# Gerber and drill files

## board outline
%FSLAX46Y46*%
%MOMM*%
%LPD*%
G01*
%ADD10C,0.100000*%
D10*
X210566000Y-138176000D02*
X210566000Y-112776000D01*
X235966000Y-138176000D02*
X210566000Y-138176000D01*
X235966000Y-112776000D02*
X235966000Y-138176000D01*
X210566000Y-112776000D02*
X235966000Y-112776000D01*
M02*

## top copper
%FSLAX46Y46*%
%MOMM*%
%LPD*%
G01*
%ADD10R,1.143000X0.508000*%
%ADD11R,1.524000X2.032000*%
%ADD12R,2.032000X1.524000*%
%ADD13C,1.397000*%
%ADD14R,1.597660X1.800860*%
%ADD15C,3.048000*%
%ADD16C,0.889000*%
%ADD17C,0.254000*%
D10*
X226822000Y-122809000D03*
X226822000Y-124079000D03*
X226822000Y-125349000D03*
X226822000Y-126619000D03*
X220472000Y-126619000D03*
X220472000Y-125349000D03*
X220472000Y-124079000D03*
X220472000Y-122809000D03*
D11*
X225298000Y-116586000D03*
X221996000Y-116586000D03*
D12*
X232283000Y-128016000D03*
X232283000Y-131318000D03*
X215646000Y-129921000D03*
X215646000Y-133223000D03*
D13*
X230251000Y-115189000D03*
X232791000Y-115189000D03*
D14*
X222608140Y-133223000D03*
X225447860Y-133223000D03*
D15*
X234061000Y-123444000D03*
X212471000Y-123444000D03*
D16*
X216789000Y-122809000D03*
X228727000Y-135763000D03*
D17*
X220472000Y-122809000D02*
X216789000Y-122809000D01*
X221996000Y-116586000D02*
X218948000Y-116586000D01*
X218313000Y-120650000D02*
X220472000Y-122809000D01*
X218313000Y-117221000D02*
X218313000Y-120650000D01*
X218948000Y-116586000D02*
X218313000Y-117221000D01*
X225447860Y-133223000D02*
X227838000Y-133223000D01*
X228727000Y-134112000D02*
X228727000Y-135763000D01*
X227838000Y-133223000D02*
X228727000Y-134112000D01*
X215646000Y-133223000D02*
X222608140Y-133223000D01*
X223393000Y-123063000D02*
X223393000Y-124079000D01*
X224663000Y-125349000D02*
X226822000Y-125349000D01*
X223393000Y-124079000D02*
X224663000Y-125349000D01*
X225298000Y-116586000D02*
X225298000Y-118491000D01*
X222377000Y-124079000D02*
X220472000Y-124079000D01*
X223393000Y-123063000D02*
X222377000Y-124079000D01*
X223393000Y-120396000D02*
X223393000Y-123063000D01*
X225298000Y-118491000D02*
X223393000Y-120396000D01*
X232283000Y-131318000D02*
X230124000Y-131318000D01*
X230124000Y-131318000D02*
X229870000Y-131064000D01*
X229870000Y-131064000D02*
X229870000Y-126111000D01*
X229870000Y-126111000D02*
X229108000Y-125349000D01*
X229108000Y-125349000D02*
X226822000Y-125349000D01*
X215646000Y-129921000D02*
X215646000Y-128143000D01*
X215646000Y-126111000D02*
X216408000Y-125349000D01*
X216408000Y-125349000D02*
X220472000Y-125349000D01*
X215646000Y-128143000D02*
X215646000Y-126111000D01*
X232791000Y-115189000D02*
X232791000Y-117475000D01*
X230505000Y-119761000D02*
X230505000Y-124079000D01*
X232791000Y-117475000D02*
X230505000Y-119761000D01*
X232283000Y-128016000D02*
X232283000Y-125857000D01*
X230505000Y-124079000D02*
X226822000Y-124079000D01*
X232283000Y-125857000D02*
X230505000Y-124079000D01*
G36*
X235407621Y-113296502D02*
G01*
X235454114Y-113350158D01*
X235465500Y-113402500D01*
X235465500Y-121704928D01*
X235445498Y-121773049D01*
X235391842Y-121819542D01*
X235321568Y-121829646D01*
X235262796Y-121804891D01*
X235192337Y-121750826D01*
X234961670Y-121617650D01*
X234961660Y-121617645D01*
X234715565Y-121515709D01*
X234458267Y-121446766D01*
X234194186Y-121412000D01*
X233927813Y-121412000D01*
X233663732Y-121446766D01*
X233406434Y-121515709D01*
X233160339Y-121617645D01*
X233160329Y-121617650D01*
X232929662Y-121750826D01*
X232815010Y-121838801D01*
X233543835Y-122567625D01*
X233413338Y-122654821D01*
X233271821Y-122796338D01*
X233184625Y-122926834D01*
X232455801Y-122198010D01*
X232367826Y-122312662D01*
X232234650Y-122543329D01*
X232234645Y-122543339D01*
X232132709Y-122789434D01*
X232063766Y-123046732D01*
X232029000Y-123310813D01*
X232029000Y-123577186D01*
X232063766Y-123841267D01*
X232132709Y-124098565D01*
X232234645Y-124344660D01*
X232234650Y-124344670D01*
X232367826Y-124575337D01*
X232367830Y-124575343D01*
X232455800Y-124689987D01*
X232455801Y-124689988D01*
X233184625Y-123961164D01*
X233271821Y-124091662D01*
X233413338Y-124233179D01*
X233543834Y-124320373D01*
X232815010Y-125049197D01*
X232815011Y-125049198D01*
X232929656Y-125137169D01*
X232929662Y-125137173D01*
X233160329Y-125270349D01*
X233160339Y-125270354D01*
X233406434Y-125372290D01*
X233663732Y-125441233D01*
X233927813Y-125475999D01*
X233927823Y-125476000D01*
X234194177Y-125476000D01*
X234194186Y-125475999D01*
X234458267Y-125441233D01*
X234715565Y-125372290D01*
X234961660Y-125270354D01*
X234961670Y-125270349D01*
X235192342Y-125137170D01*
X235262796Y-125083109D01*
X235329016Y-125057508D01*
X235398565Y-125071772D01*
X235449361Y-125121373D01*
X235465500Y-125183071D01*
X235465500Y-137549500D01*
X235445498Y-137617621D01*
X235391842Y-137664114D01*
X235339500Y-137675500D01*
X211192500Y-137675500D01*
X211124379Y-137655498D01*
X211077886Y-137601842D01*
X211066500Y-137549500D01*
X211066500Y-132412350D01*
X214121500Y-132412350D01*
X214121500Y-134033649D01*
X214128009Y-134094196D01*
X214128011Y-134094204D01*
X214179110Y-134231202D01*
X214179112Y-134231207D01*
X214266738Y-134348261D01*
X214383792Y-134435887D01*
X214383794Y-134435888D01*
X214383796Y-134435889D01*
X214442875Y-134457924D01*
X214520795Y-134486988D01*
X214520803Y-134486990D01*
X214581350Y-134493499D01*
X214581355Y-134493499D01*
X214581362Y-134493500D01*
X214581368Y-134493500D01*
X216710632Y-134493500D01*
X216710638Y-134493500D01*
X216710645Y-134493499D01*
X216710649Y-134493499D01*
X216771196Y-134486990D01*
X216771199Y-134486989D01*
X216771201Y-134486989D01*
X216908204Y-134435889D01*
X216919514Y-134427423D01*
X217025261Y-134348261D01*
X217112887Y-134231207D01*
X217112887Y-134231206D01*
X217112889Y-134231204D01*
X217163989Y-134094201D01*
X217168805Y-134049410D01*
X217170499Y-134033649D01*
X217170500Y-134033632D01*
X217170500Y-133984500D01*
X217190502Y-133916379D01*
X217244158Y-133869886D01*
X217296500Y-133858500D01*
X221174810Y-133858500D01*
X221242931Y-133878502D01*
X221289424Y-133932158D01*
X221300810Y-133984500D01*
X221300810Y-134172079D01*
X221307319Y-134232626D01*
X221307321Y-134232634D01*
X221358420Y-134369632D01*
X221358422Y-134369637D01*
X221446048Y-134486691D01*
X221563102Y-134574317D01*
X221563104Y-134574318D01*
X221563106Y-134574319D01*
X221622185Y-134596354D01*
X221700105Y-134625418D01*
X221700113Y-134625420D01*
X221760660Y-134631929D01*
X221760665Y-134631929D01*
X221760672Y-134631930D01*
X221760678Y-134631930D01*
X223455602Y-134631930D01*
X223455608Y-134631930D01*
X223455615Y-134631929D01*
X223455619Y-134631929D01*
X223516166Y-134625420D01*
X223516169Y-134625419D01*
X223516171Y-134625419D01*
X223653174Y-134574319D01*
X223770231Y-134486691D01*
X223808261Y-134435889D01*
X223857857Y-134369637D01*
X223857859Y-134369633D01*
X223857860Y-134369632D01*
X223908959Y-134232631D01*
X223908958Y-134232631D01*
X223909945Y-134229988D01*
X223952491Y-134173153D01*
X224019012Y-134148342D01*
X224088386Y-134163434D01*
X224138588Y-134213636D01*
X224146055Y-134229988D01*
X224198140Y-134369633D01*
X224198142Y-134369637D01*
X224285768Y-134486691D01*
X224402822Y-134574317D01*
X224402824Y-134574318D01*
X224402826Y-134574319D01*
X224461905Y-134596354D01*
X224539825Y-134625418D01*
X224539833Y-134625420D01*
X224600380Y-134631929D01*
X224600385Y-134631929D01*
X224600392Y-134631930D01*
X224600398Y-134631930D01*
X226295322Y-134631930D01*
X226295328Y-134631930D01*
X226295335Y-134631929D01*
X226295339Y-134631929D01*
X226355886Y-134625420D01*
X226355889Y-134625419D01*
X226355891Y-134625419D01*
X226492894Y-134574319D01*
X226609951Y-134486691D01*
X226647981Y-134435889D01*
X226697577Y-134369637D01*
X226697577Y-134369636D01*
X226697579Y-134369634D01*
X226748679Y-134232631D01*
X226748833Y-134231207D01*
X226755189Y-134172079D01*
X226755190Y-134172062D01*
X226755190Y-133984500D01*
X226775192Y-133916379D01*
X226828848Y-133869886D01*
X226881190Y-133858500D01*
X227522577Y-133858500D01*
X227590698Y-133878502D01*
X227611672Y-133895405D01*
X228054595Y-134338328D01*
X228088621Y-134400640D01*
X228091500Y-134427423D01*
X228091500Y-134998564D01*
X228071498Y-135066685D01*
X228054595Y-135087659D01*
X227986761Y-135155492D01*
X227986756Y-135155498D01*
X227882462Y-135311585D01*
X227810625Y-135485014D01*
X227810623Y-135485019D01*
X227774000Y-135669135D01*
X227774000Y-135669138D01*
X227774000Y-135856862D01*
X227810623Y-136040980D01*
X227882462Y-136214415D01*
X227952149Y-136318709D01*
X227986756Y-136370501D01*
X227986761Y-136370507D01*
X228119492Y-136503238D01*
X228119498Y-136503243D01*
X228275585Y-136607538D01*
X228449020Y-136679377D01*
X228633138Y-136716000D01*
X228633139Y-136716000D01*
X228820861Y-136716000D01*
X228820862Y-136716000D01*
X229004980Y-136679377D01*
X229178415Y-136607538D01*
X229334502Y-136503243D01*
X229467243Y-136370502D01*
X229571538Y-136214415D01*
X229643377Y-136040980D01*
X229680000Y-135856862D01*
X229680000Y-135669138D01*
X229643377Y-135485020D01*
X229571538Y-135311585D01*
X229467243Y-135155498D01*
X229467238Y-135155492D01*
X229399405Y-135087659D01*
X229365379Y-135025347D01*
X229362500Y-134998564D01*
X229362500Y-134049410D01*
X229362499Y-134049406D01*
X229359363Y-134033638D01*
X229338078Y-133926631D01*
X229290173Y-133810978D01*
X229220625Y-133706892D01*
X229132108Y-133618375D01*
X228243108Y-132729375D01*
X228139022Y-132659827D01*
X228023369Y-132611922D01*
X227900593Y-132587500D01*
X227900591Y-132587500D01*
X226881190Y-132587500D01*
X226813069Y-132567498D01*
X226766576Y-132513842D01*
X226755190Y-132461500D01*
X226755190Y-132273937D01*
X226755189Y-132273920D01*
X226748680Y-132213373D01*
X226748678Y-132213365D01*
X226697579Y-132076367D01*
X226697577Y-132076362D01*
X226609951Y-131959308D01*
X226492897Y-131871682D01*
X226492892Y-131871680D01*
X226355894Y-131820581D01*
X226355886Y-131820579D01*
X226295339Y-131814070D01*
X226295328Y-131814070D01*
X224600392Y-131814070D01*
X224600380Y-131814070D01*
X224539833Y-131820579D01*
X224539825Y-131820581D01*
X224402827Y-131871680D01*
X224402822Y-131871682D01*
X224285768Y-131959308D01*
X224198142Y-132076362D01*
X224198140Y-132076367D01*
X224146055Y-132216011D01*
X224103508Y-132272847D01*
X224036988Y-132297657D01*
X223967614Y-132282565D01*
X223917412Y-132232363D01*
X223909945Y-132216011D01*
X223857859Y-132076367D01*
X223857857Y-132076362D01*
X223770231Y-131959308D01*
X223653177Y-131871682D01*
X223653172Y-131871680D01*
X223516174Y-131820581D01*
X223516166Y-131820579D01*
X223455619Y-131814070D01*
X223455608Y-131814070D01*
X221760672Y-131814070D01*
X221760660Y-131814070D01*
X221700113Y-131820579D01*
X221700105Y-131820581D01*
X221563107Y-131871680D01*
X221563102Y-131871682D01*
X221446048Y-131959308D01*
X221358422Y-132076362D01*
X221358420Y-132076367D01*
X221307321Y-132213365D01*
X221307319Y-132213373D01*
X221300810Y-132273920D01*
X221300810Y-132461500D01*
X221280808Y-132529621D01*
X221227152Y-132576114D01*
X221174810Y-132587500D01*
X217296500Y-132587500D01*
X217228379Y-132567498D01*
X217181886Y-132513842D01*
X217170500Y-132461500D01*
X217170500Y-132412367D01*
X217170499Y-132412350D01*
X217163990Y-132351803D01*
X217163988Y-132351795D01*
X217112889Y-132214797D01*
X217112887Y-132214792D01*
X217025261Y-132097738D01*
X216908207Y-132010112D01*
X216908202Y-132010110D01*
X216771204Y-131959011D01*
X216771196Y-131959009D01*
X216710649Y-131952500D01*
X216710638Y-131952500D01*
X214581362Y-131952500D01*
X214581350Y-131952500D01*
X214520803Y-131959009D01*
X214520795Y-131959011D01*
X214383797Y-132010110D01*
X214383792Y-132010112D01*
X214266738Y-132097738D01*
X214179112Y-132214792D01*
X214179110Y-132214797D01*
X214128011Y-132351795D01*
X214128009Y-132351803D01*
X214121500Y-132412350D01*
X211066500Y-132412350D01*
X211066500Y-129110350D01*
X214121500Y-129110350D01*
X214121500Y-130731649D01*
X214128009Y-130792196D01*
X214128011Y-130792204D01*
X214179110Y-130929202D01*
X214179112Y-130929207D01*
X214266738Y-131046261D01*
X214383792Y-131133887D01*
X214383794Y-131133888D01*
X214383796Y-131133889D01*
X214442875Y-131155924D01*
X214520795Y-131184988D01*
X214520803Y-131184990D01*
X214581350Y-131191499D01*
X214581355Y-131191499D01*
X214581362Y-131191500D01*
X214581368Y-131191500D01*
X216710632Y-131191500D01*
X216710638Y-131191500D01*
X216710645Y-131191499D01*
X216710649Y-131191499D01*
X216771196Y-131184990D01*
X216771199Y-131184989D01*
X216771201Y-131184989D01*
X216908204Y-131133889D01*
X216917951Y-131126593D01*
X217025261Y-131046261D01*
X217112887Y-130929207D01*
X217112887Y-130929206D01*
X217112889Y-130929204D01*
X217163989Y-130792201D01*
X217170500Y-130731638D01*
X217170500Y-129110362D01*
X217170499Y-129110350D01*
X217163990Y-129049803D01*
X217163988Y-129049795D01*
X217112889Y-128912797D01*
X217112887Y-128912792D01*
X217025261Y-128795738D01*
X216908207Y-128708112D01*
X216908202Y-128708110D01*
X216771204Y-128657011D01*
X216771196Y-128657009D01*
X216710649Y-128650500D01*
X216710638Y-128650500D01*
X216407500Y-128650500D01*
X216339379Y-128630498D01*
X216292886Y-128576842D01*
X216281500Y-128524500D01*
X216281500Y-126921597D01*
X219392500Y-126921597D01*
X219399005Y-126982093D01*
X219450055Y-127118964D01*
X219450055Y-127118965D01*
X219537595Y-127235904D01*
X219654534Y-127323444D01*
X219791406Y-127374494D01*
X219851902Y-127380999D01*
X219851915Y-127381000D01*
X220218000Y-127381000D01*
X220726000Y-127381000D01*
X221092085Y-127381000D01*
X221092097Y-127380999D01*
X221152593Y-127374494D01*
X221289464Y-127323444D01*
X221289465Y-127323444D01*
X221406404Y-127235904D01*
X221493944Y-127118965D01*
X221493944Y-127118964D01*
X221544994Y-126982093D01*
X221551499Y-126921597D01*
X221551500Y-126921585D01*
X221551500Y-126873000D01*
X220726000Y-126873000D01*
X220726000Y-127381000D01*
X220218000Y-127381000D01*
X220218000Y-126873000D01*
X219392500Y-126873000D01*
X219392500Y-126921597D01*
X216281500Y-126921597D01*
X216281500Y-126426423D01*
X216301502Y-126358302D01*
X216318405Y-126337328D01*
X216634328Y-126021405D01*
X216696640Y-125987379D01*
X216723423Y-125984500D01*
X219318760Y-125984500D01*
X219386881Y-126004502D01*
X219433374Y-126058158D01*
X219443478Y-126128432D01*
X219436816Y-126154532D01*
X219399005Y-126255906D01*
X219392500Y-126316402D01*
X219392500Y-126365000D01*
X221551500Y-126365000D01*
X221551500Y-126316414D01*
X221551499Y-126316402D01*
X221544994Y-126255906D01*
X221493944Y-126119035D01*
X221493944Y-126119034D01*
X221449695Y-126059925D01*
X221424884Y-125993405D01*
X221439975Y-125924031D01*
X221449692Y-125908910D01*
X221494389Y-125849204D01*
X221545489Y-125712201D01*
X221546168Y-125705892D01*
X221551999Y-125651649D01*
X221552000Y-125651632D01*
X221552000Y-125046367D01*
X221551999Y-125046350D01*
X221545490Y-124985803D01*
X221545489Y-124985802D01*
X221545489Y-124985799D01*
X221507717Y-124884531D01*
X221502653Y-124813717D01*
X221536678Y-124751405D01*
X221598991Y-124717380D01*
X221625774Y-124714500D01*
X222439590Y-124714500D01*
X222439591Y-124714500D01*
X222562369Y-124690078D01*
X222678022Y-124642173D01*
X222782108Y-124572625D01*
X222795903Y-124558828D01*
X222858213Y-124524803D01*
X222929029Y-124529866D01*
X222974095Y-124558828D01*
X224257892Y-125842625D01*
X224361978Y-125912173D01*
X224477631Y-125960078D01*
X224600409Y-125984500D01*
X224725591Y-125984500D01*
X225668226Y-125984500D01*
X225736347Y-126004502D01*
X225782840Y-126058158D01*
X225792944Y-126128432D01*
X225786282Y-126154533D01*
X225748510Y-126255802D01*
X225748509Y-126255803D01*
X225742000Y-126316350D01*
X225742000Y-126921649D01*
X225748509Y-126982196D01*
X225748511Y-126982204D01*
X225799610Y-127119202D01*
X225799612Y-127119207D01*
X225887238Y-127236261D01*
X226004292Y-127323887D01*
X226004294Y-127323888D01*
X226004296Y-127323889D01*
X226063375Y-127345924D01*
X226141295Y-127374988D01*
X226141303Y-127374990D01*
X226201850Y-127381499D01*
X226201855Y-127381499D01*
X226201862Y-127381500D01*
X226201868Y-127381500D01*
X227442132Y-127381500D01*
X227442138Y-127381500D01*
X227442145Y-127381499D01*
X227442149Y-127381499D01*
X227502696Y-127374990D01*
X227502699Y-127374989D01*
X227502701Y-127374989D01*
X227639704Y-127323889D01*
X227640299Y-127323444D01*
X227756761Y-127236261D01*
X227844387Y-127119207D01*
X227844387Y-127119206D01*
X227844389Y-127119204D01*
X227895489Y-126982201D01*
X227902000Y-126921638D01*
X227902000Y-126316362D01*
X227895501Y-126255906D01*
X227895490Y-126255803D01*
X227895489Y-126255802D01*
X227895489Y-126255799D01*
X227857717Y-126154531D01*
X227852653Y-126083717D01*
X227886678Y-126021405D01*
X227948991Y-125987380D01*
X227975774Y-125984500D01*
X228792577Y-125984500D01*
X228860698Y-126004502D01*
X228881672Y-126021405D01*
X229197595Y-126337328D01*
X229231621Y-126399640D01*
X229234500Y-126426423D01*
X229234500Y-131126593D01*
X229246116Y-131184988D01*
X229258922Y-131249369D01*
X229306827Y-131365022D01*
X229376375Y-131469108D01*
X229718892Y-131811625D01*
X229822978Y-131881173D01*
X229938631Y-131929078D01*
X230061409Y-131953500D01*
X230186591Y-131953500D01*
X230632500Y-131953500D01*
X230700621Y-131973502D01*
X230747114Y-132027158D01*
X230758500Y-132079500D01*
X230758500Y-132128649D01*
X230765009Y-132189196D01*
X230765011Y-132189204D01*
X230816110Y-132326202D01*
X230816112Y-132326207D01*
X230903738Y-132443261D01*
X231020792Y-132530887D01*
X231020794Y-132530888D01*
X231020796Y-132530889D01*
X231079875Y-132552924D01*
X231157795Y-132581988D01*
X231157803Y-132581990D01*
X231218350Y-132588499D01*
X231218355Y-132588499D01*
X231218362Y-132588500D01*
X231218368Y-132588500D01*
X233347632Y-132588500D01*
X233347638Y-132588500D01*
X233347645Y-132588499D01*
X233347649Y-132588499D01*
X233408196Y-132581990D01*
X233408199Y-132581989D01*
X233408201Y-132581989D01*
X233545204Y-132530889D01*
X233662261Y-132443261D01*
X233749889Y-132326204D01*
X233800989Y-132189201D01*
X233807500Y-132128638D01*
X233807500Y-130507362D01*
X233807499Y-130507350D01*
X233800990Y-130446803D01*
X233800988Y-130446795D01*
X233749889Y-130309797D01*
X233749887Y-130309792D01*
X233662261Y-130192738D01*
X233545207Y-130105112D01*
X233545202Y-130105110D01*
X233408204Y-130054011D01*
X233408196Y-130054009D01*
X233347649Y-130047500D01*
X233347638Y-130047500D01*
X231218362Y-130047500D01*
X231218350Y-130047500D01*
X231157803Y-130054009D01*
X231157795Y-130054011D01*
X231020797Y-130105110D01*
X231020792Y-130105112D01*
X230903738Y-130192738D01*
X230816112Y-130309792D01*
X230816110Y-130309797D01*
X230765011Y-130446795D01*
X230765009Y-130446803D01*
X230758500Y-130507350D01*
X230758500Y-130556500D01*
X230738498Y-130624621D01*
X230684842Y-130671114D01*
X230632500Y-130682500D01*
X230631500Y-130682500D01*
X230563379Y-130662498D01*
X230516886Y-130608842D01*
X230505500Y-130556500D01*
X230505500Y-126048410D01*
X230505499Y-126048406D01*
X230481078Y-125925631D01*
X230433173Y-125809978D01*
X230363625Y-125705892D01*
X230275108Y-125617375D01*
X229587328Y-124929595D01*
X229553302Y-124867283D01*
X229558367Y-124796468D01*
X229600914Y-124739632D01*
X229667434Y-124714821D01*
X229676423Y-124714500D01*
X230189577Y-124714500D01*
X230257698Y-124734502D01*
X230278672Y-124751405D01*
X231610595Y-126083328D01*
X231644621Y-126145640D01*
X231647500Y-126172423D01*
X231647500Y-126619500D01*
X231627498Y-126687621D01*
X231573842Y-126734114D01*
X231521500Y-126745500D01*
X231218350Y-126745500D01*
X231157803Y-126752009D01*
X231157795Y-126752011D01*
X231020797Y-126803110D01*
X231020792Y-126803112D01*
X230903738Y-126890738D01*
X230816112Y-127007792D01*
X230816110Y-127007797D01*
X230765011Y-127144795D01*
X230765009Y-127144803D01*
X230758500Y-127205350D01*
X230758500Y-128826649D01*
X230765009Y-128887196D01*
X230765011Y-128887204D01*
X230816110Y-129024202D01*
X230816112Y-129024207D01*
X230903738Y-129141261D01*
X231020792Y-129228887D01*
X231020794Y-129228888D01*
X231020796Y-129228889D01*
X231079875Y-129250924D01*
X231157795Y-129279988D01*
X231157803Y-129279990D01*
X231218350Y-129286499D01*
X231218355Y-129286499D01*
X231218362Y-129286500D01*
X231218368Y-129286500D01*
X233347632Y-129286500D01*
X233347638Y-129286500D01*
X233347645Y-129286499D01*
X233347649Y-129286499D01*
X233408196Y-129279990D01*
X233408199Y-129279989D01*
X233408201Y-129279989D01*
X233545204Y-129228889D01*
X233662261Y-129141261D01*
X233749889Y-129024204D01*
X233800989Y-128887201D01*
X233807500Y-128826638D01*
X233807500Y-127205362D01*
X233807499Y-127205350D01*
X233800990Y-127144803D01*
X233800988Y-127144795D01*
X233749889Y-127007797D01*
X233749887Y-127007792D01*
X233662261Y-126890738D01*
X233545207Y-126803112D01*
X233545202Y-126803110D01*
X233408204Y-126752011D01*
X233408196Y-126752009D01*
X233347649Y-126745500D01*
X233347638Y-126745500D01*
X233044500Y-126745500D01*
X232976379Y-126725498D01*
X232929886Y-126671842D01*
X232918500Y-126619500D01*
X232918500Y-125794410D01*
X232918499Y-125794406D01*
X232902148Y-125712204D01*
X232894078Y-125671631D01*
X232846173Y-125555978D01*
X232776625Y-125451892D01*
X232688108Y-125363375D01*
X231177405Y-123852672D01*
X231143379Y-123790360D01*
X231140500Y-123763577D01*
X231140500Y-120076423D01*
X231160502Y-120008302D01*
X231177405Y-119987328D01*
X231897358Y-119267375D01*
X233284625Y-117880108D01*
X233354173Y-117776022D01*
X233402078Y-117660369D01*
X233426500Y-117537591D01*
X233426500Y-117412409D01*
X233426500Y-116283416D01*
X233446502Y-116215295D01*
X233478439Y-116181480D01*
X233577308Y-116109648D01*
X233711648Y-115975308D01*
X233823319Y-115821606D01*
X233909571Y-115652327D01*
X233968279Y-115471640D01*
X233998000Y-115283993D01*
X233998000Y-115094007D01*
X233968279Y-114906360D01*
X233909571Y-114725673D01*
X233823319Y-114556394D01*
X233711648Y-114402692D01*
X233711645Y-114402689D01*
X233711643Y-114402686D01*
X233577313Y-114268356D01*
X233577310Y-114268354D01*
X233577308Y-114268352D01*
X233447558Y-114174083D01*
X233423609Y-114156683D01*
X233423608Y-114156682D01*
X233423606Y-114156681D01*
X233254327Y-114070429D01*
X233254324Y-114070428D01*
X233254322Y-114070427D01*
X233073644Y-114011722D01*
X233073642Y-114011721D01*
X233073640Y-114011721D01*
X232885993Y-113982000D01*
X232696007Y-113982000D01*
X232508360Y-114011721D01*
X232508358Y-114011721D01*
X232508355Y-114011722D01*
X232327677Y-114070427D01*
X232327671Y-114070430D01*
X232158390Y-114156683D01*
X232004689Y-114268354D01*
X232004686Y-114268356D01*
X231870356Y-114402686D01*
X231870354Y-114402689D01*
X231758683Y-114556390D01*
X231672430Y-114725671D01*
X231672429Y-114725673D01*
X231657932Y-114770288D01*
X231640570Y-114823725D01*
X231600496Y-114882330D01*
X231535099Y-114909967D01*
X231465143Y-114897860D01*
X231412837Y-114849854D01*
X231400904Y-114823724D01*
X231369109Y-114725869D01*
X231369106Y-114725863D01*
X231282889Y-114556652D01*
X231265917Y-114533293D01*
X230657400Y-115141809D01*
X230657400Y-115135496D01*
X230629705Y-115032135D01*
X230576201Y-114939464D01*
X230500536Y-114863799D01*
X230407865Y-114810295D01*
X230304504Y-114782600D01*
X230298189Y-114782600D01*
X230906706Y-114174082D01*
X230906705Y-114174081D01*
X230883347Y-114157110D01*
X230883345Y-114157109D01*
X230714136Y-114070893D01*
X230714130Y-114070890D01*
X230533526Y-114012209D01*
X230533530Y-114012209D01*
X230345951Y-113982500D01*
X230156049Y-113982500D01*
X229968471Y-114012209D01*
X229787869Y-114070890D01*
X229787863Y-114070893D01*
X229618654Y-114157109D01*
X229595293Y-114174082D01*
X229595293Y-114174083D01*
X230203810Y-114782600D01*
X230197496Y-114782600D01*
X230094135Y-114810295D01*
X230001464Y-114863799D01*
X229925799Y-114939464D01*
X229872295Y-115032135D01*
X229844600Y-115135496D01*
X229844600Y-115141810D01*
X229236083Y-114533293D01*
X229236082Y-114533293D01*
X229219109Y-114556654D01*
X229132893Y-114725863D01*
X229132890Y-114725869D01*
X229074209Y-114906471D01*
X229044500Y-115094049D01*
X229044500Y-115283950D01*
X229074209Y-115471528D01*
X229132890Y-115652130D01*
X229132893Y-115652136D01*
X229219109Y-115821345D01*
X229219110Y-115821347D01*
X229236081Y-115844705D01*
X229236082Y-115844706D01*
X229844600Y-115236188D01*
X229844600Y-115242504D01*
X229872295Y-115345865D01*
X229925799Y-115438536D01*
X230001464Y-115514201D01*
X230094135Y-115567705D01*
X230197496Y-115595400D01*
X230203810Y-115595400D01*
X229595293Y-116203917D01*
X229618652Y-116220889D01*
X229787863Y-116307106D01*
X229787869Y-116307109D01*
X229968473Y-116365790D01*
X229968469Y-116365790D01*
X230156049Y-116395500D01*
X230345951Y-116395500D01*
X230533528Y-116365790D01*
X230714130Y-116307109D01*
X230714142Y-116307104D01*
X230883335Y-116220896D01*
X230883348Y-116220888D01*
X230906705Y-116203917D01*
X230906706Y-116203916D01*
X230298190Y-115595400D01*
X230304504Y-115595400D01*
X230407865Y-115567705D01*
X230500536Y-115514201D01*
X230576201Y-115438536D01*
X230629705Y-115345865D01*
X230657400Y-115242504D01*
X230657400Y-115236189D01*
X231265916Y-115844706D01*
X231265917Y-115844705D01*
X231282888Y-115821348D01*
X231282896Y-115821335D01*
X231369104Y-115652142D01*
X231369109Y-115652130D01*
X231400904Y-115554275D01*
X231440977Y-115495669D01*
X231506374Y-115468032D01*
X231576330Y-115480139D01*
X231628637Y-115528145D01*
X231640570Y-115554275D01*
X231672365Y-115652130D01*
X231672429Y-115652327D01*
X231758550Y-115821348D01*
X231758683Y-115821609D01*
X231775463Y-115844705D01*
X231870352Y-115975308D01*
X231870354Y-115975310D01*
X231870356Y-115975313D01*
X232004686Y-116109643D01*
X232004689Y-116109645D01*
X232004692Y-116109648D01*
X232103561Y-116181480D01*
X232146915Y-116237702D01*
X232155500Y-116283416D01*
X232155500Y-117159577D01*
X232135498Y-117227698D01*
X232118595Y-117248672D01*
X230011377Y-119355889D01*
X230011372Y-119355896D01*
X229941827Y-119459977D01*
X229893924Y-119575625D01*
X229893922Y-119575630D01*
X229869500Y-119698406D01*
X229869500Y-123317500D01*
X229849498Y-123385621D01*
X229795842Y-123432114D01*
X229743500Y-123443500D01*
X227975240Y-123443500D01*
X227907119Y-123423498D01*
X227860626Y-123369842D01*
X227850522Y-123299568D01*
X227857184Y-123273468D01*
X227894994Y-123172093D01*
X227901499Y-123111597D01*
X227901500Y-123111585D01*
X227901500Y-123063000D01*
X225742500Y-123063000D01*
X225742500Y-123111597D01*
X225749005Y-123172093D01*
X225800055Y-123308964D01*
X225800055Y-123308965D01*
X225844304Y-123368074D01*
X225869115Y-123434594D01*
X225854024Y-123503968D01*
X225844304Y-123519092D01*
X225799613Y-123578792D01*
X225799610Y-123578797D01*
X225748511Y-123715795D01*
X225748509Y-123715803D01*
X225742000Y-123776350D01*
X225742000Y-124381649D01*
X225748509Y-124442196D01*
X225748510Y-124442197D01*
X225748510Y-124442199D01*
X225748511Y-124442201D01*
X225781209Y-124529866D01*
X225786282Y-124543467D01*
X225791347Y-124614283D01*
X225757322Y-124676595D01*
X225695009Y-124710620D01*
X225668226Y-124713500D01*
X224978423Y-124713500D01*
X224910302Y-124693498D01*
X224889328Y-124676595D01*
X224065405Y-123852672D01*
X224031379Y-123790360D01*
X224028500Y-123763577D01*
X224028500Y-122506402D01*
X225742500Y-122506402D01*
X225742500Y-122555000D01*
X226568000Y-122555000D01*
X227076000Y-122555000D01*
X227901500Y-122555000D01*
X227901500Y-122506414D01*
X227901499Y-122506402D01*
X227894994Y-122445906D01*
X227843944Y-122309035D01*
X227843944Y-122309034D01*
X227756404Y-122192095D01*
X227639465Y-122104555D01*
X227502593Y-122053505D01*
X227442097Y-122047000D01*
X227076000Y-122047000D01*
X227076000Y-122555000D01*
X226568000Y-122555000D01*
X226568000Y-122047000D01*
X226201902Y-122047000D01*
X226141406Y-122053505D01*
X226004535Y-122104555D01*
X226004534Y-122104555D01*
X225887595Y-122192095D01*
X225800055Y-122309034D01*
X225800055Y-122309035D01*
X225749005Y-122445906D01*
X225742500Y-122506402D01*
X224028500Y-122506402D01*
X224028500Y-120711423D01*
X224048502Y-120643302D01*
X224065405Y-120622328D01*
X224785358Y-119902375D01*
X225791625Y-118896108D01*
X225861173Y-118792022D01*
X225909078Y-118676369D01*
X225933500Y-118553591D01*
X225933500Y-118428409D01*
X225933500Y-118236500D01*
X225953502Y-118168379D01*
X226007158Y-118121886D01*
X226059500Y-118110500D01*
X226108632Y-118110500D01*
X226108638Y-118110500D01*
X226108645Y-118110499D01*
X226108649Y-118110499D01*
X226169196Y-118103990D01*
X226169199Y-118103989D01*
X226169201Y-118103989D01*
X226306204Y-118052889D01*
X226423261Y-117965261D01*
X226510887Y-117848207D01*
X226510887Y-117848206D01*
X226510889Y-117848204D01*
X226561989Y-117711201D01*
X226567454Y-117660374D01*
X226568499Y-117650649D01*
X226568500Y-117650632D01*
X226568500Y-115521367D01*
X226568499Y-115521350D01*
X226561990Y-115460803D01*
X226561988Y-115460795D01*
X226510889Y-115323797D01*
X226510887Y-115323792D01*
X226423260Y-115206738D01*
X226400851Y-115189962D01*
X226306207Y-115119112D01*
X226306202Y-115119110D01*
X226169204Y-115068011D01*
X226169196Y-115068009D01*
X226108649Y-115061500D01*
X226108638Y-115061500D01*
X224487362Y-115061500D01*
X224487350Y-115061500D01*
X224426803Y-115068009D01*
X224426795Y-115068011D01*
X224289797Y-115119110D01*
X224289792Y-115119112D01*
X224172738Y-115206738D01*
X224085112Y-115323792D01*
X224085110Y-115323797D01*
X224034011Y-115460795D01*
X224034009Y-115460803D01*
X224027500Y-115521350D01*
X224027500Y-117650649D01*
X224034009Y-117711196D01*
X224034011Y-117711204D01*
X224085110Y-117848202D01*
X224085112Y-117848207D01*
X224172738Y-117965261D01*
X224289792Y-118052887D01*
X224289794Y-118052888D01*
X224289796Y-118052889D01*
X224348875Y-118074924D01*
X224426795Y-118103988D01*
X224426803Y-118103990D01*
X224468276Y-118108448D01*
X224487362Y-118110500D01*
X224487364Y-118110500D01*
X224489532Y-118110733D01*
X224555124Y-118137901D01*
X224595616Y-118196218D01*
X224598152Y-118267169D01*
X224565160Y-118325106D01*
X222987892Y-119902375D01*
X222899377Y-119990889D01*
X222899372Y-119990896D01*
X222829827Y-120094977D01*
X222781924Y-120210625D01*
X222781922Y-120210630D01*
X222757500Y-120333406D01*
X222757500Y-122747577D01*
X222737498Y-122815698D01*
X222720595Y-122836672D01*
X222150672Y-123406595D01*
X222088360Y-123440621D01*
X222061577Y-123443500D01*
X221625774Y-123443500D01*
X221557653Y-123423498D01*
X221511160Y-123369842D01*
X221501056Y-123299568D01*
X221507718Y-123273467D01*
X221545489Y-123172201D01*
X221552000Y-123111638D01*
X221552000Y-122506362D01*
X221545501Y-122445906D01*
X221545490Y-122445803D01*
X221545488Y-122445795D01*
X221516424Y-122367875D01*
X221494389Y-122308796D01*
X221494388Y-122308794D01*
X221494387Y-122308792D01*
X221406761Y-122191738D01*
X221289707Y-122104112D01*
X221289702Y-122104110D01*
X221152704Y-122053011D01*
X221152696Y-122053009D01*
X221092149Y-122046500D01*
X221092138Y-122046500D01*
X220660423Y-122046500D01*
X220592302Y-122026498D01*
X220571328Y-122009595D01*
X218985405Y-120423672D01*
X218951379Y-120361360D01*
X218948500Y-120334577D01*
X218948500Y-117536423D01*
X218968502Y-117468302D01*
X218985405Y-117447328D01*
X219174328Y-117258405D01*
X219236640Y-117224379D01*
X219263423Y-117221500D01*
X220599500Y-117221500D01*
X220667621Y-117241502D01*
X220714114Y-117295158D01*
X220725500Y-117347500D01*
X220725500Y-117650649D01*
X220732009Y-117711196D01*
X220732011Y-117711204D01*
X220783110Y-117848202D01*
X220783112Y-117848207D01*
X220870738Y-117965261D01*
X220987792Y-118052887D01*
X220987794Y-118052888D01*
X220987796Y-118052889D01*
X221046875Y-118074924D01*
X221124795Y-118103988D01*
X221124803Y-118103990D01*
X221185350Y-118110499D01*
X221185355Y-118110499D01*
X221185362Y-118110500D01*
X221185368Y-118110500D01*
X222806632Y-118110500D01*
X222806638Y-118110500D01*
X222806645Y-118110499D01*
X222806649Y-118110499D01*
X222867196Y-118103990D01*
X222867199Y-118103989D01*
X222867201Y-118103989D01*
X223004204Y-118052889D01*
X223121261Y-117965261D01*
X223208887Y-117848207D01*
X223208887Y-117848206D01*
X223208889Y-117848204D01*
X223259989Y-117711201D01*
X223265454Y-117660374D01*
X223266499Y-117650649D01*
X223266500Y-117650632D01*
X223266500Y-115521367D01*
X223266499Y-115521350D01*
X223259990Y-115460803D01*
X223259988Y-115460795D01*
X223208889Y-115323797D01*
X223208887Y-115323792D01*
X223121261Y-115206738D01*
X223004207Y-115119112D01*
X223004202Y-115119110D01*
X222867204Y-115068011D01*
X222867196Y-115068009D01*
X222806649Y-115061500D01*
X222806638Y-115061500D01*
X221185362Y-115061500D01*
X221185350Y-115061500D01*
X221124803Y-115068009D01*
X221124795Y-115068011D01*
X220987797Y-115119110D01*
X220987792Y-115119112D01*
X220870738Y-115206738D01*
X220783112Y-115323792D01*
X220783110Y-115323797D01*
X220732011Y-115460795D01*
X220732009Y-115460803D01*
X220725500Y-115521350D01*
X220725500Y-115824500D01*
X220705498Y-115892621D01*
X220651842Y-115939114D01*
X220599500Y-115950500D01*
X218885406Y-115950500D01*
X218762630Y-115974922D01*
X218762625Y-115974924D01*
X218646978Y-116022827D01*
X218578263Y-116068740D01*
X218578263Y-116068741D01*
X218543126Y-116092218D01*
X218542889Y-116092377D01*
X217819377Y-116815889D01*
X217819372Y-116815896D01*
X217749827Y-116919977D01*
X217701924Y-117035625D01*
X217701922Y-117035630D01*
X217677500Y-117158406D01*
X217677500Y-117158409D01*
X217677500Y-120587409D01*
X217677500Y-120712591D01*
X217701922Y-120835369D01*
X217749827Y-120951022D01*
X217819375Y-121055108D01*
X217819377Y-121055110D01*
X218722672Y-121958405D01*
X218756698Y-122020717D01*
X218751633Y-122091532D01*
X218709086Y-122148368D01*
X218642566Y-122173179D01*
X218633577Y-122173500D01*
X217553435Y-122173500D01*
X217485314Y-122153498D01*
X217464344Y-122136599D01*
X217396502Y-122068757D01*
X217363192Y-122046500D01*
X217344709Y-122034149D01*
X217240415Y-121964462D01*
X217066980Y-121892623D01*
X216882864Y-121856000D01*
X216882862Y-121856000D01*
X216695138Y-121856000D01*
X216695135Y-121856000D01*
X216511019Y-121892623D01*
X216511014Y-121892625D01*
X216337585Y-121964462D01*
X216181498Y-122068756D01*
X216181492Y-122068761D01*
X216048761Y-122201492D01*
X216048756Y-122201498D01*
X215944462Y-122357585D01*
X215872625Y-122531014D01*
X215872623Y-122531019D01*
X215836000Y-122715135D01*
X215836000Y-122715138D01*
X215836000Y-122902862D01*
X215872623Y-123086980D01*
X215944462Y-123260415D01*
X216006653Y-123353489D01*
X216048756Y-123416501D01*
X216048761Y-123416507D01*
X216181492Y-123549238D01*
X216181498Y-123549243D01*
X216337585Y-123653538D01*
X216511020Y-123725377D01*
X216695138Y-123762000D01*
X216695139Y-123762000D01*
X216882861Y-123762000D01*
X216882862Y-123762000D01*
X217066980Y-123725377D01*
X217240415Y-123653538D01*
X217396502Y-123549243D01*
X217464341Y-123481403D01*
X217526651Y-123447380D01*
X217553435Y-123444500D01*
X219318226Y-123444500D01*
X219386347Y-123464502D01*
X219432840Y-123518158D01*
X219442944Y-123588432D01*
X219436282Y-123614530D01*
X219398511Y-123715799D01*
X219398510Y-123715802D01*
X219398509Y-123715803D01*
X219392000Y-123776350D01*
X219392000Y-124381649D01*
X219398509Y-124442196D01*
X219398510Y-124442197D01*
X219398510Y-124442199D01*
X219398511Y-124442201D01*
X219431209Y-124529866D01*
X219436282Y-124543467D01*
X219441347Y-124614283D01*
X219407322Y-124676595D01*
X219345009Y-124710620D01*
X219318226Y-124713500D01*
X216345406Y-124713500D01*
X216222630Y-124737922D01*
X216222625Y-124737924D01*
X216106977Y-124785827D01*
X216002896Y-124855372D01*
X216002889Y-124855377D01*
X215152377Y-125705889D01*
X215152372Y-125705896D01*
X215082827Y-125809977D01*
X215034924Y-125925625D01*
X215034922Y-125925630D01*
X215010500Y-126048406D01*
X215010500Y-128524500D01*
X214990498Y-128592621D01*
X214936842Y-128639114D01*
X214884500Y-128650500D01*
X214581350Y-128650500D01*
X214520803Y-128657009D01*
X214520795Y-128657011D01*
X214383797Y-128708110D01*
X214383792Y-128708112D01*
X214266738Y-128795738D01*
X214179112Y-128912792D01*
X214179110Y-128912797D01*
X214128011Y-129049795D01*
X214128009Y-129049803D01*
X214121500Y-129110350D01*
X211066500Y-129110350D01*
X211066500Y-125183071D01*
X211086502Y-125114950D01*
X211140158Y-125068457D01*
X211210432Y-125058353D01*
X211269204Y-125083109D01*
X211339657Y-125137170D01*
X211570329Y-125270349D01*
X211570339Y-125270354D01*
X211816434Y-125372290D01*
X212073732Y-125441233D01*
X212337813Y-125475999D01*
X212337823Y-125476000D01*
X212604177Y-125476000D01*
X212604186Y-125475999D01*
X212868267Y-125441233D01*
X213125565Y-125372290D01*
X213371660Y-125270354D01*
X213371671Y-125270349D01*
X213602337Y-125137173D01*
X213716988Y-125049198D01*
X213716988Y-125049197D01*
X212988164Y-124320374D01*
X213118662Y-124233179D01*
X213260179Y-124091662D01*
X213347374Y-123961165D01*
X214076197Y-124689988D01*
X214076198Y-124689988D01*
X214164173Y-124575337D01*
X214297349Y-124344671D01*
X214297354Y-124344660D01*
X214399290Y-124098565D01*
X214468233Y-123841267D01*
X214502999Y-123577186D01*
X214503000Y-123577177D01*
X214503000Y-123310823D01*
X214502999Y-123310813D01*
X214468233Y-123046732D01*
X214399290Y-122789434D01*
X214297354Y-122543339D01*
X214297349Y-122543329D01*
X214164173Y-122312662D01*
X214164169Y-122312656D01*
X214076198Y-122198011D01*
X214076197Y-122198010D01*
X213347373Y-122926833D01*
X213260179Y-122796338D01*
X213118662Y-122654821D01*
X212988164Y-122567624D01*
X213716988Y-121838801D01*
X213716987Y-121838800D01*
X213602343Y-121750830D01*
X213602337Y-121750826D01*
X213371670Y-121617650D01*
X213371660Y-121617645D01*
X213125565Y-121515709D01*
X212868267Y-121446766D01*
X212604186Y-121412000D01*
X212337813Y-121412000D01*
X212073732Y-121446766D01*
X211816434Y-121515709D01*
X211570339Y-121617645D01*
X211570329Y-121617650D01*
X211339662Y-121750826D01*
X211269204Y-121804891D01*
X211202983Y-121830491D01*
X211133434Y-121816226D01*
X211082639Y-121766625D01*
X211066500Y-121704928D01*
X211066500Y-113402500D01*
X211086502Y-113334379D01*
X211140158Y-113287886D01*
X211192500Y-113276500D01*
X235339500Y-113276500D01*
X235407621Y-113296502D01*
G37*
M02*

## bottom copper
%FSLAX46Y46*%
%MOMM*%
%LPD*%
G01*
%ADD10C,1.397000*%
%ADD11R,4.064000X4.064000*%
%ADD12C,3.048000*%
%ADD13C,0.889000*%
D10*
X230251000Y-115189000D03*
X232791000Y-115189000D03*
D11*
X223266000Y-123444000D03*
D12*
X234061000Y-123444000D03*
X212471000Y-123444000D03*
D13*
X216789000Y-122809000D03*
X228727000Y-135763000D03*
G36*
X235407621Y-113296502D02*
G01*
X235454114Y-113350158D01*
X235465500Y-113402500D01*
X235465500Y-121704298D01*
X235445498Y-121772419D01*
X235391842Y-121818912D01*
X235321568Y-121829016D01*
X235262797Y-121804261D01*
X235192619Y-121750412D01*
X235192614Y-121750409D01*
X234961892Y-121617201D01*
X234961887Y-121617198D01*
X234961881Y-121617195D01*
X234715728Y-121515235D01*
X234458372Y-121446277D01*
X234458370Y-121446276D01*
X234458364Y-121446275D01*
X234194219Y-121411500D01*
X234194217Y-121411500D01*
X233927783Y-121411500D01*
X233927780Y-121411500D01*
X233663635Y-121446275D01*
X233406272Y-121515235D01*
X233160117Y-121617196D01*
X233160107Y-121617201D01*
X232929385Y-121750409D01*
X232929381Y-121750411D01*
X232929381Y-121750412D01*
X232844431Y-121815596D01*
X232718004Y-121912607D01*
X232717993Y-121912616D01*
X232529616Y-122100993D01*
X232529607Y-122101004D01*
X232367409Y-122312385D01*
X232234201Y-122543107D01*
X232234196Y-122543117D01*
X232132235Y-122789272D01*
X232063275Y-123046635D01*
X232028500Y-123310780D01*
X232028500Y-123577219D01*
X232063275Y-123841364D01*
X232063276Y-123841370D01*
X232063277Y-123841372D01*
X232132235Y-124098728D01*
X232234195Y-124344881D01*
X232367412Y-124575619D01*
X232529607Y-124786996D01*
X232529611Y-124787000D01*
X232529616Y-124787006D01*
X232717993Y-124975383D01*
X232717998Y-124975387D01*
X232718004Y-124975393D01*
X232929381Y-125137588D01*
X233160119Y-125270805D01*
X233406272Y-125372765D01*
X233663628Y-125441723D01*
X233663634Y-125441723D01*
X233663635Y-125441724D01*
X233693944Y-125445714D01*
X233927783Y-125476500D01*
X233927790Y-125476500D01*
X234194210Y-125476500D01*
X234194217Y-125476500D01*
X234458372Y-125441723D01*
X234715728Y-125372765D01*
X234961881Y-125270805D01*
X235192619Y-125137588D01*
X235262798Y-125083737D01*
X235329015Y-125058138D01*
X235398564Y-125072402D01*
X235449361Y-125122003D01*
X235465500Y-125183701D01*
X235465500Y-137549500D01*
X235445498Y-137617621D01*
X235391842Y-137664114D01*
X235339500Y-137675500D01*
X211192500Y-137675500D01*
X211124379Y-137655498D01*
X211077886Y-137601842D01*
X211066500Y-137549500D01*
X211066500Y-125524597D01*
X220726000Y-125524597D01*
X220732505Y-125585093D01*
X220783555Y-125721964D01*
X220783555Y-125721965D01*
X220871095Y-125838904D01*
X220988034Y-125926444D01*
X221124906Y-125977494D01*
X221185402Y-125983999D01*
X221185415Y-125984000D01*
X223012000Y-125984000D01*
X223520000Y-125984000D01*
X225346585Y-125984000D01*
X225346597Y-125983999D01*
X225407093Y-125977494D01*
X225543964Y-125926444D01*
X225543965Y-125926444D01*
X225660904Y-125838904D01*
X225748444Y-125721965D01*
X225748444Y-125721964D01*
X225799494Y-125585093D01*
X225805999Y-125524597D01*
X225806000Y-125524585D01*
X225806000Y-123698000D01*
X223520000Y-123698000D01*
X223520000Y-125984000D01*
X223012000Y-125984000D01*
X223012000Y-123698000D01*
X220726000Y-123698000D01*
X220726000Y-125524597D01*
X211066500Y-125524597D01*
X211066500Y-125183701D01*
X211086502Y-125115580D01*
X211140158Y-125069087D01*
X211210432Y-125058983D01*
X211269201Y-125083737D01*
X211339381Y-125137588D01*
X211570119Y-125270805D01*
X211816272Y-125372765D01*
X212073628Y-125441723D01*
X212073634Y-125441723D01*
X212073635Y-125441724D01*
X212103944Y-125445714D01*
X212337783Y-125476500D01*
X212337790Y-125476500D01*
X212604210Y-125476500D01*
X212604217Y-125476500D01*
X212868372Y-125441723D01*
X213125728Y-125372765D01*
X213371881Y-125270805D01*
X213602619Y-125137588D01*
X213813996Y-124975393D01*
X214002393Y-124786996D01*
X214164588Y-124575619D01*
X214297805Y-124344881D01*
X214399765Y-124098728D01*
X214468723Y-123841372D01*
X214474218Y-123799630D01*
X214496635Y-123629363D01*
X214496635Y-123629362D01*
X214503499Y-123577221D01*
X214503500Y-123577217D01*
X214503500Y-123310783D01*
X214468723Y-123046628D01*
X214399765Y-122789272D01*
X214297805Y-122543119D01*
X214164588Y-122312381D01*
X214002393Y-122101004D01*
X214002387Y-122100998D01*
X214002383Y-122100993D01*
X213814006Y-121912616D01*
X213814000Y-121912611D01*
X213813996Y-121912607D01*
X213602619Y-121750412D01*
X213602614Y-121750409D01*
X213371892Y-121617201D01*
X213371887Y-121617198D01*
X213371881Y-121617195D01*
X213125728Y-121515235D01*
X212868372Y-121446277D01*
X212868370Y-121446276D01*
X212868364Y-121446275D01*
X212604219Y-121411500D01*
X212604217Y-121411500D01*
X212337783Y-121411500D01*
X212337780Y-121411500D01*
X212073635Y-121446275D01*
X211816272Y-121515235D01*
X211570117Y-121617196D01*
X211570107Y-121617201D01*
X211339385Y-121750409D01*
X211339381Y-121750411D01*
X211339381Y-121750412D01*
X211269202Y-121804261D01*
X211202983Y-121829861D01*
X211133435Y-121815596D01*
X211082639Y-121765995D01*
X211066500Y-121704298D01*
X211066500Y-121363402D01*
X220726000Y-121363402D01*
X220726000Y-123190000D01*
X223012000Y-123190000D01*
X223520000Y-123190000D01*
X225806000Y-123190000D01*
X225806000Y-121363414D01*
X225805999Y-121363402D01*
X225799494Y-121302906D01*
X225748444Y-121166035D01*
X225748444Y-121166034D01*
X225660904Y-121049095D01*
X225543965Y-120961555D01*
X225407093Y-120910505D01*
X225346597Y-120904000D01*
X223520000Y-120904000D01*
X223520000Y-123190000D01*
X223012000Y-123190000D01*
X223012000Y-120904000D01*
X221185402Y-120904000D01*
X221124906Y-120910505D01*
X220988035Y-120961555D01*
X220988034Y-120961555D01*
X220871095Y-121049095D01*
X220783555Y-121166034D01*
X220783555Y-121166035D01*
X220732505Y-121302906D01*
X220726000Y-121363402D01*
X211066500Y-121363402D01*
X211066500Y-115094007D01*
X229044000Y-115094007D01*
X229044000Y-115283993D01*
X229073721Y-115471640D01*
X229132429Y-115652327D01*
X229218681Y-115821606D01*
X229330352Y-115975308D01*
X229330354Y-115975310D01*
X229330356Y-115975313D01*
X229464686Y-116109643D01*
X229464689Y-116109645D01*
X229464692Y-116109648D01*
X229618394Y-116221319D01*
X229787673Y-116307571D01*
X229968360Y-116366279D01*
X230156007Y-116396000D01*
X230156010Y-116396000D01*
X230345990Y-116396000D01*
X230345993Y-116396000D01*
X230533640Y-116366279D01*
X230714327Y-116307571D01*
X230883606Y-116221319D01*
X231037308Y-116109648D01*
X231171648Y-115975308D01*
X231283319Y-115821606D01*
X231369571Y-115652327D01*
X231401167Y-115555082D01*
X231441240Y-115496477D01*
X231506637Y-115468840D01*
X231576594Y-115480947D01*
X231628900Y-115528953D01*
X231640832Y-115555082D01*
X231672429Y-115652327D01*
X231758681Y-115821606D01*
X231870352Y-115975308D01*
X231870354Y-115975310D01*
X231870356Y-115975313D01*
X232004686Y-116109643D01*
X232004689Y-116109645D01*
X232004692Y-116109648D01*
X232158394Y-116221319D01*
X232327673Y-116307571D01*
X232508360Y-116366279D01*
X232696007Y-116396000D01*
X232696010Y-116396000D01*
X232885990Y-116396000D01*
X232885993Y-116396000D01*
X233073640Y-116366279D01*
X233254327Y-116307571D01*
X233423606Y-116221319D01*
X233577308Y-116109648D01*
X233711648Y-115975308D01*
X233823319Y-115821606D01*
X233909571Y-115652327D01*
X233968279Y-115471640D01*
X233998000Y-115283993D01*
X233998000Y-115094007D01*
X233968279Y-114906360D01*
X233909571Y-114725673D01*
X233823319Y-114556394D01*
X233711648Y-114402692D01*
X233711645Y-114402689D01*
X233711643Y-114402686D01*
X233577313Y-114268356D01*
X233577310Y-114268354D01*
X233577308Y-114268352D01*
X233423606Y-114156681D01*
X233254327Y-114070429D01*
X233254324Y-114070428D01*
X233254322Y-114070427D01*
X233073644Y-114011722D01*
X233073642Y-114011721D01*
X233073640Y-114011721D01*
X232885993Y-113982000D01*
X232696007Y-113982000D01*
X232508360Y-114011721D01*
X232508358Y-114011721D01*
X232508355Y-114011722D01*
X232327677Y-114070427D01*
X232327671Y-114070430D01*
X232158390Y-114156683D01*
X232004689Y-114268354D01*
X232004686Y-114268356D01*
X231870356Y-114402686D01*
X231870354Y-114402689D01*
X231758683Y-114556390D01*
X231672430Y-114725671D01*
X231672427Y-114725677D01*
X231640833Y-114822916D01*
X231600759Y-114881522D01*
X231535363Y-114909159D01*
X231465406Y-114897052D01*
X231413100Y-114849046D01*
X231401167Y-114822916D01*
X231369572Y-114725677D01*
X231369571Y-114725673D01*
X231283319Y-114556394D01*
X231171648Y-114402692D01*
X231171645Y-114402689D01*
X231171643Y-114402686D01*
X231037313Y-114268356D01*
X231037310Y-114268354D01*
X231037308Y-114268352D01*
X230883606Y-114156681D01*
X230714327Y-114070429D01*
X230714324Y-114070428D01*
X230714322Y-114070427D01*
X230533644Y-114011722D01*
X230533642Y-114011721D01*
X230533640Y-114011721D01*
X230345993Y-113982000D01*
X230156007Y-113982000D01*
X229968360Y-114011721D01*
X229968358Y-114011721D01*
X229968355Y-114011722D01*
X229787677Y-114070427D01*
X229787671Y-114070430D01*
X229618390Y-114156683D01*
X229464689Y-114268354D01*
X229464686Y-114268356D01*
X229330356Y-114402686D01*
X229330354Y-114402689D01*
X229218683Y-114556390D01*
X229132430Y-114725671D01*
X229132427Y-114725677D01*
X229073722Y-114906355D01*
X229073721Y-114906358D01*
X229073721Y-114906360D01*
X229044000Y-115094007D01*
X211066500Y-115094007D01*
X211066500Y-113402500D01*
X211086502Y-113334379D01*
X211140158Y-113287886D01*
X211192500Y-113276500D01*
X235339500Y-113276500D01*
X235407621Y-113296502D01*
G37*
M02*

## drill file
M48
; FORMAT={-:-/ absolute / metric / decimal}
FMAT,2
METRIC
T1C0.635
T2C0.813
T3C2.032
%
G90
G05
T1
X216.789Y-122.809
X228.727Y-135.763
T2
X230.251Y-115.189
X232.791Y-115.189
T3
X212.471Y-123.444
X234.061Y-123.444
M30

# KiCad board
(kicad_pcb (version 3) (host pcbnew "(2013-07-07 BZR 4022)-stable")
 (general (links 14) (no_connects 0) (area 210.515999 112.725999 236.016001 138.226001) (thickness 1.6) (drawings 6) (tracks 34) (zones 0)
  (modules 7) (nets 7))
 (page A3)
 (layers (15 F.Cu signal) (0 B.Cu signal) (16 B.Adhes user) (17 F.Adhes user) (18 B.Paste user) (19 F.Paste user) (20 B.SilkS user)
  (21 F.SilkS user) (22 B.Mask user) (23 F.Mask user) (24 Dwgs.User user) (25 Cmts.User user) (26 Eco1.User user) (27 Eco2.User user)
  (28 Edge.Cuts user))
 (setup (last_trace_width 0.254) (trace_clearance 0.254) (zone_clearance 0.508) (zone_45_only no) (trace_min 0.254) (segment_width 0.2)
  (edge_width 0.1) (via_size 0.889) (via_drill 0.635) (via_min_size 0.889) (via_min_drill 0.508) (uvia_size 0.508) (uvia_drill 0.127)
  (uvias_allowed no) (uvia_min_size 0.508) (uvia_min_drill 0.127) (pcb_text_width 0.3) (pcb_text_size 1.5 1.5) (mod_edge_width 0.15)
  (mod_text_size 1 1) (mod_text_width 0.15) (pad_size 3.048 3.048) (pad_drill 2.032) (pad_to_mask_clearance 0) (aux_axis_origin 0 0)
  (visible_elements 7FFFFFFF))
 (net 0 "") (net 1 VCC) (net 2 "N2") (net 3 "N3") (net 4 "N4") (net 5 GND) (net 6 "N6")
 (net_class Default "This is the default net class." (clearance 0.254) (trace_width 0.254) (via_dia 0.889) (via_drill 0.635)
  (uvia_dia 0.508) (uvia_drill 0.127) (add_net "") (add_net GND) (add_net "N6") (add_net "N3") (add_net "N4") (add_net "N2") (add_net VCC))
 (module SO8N (layer F.Cu) (at 223.647 124.714 270)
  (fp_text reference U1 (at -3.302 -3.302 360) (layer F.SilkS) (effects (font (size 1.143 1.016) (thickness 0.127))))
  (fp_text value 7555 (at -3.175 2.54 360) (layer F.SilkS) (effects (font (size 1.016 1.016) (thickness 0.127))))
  (pad 8 smd rect (at -1.905 -3.175 270) (size 0.508 1.143) (layers F.Cu F.Paste F.Mask) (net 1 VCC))
  (pad 7 smd rect (at -0.635 -3.175 270) (size 0.508 1.143) (layers F.Cu F.Paste F.Mask) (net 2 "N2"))
  (pad 6 smd rect (at 0.635 -3.175 270) (size 0.508 1.143) (layers F.Cu F.Paste F.Mask) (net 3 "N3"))
  (pad 5 smd rect (at 1.905 -3.175 270) (size 0.508 1.143) (layers F.Cu F.Paste F.Mask))
  (pad 4 smd rect (at 1.905 3.175 270) (size 0.508 1.143) (layers F.Cu F.Paste F.Mask) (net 1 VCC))
  (pad 3 smd rect (at 0.635 3.175 270) (size 0.508 1.143) (layers F.Cu F.Paste F.Mask) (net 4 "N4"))
  (pad 2 smd rect (at -0.635 3.175 270) (size 0.508 1.143) (layers F.Cu F.Paste F.Mask) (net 3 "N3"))
  (pad 1 smd rect (at -1.905 3.175 270) (size 0.508 1.143) (layers F.Cu F.Paste F.Mask) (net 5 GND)))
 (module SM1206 (layer F.Cu) (at 223.647 116.586 180)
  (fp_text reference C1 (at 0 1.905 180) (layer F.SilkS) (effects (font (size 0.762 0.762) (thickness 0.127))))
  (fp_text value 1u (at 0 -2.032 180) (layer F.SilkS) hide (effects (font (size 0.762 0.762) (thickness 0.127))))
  (pad 1 smd rect (at -1.651 0 180) (size 1.524 2.032) (layers F.Cu F.Paste F.Mask) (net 3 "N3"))
  (pad 2 smd rect (at 1.651 0 180) (size 1.524 2.032) (layers F.Cu F.Paste F.Mask) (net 5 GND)))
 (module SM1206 (layer F.Cu) (at 232.283 129.667 270)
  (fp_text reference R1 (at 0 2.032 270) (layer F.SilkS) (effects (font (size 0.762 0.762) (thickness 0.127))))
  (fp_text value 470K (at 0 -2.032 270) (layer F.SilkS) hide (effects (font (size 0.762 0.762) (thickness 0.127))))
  (pad 1 smd rect (at -1.651 0 270) (size 1.524 2.032) (layers F.Cu F.Paste F.Mask) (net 2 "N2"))
  (pad 2 smd rect (at 1.651 0 270) (size 1.524 2.032) (layers F.Cu F.Paste F.Mask) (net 3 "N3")))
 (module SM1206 (layer F.Cu) (at 215.646 131.572 270)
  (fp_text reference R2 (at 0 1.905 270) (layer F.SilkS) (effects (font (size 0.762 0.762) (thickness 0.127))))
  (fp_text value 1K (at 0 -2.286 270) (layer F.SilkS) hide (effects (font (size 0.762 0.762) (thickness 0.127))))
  (pad 1 smd rect (at -1.651 0 270) (size 1.524 2.032) (layers F.Cu F.Paste F.Mask) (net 4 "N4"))
  (pad 2 smd rect (at 1.651 0 270) (size 1.524 2.032) (layers F.Cu F.Paste F.Mask) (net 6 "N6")))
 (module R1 (layer F.Cu) (at 231.521 115.189) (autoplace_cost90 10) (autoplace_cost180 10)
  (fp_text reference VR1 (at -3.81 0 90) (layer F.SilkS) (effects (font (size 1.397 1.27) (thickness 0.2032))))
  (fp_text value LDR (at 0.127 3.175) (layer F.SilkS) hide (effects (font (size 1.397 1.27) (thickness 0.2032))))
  (pad 1 thru_hole circle (at -1.27 0) (size 1.397 1.397) (drill 0.8128) (layers *.Cu *.Mask F.SilkS) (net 1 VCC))
  (pad 2 thru_hole circle (at 1.27 0) (size 1.397 1.397) (drill 0.8128) (layers *.Cu *.Mask F.SilkS) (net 2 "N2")))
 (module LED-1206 (layer F.Cu) (at 224.028 133.223)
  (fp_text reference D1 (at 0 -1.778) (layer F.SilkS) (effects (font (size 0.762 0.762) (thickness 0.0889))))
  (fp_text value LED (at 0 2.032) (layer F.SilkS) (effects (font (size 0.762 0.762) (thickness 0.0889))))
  (pad 1 smd rect (at -1.41986 0) (size 1.59766 1.80086) (layers F.Cu F.Paste F.Mask) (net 6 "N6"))
  (pad 2 smd rect (at 1.41986 0) (size 1.59766 1.80086) (layers F.Cu F.Paste F.Mask) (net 5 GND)))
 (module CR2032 (layer B.Cu) (at 223.266 123.444 180)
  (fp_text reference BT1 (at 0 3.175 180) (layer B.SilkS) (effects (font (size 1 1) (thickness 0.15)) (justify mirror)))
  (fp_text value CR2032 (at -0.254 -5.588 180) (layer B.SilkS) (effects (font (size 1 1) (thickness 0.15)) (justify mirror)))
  (pad 2 smd rect (at 0 0 180) (size 4.064 4.064) (layers B.Cu B.Paste B.Mask) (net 5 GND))
  (pad 1 thru_hole circle (at -10.795 0 180) (size 3.048 3.048) (drill 2.032) (layers *.Cu *.Mask B.SilkS) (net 1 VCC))
  (pad 1 thru_hole circle (at 10.795 0 180) (size 3.048 3.048) (drill 2.032) (layers *.Cu *.Mask B.SilkS) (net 1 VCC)))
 (gr_line (start 210.566 138.176) (end 210.566 112.776) (angle 90) (layer Edge.Cuts) (width 0.1))
 (gr_line (start 235.966 138.176) (end 210.566 138.176) (angle 90) (layer Edge.Cuts) (width 0.1))
 (gr_line (start 235.966 112.776) (end 235.966 138.176) (angle 90) (layer Edge.Cuts) (width 0.1))
 (gr_line (start 210.566 112.776) (end 235.966 112.776) (angle 90) (layer Edge.Cuts) (width 0.1))
 (segment (start 220.472 122.809) (end 216.789 122.809) (width 0.254) (layer F.Cu) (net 5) (status 400000))
 (via (at 216.789 122.809) (size 0.889) (layers F.Cu B.Cu) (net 5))
 (segment (start 221.996 116.586) (end 218.948 116.586) (width 0.254) (layer F.Cu) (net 5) (status 400000))
 (segment (start 218.313 120.65) (end 220.472 122.809) (width 0.254) (layer F.Cu) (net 5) (status 800000))
 (segment (start 218.313 117.221) (end 218.313 120.65) (width 0.254) (layer F.Cu) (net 5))
 (segment (start 218.948 116.586) (end 218.313 117.221) (width 0.254) (layer F.Cu) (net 5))
 (segment (start 225.44786 133.223) (end 227.838 133.223) (width 0.254) (layer F.Cu) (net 5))
 (via (at 228.727 135.763) (size 0.889) (layers F.Cu B.Cu) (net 5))
 (segment (start 228.727 134.112) (end 228.727 135.763) (width 0.254) (layer F.Cu) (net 5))
 (segment (start 227.838 133.223) (end 228.727 134.112) (width 0.254) (layer F.Cu) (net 5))
 (segment (start 215.646 133.223) (end 222.60814 133.223) (width 0.254) (layer F.Cu) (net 6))
 (segment (start 223.393 123.063) (end 223.393 124.079) (width 0.254) (layer F.Cu) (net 3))
 (segment (start 224.663 125.349) (end 226.822 125.349) (width 0.254) (layer F.Cu) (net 3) (status 800000))
 (segment (start 223.393 124.079) (end 224.663 125.349) (width 0.254) (layer F.Cu) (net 3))
 (segment (start 225.298 116.586) (end 225.298 118.491) (width 0.254) (layer F.Cu) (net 3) (status 400000))
 (segment (start 222.377 124.079) (end 220.472 124.079) (width 0.254) (layer F.Cu) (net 3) (status 800000))
 (segment (start 223.393 123.063) (end 222.377 124.079) (width 0.254) (layer F.Cu) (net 3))
 (segment (start 223.393 120.396) (end 223.393 123.063) (width 0.254) (layer F.Cu) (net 3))
 (segment (start 225.298 118.491) (end 223.393 120.396) (width 0.254) (layer F.Cu) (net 3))
 (segment (start 232.283 131.318) (end 230.124 131.318) (width 0.254) (layer F.Cu) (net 3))
 (segment (start 230.124 131.318) (end 229.87 131.064) (width 0.254) (layer F.Cu) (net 3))
 (segment (start 229.87 131.064) (end 229.87 126.111) (width 0.254) (layer F.Cu) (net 3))
 (segment (start 229.87 126.111) (end 229.108 125.349) (width 0.254) (layer F.Cu) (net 3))
 (segment (start 229.108 125.349) (end 226.822 125.349) (width 0.254) (layer F.Cu) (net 3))
 (segment (start 215.646 129.921) (end 215.646 128.143) (width 0.254) (layer F.Cu) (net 4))
 (segment (start 215.646 126.111) (end 216.408 125.349) (width 0.254) (layer F.Cu) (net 4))
 (segment (start 216.408 125.349) (end 220.472 125.349) (width 0.254) (layer F.Cu) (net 4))
 (segment (start 215.646 128.143) (end 215.646 126.111) (width 0.254) (layer F.Cu) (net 4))
 (segment (start 232.791 115.189) (end 232.791 117.475) (width 0.254) (layer F.Cu) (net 2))
 (segment (start 230.505 119.761) (end 230.505 124.079) (width 0.254) (layer F.Cu) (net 2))
 (segment (start 232.791 117.475) (end 230.505 119.761) (width 0.254) (layer F.Cu) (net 2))
 (segment (start 232.283 128.016) (end 232.283 125.857) (width 0.254) (layer F.Cu) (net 2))
 (segment (start 230.505 124.079) (end 226.822 124.079) (width 0.254) (layer F.Cu) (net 2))
 (segment (start 232.283 125.857) (end 230.505 124.079) (width 0.254) (layer F.Cu) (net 2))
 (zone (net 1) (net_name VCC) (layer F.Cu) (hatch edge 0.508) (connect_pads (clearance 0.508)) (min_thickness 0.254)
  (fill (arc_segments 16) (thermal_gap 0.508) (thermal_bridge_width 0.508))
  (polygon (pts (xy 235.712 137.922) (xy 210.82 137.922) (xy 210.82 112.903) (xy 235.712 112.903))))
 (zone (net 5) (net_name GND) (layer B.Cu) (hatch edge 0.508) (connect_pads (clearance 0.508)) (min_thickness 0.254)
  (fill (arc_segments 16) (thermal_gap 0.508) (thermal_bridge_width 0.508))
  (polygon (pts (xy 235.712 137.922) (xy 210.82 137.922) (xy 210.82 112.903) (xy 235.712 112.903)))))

